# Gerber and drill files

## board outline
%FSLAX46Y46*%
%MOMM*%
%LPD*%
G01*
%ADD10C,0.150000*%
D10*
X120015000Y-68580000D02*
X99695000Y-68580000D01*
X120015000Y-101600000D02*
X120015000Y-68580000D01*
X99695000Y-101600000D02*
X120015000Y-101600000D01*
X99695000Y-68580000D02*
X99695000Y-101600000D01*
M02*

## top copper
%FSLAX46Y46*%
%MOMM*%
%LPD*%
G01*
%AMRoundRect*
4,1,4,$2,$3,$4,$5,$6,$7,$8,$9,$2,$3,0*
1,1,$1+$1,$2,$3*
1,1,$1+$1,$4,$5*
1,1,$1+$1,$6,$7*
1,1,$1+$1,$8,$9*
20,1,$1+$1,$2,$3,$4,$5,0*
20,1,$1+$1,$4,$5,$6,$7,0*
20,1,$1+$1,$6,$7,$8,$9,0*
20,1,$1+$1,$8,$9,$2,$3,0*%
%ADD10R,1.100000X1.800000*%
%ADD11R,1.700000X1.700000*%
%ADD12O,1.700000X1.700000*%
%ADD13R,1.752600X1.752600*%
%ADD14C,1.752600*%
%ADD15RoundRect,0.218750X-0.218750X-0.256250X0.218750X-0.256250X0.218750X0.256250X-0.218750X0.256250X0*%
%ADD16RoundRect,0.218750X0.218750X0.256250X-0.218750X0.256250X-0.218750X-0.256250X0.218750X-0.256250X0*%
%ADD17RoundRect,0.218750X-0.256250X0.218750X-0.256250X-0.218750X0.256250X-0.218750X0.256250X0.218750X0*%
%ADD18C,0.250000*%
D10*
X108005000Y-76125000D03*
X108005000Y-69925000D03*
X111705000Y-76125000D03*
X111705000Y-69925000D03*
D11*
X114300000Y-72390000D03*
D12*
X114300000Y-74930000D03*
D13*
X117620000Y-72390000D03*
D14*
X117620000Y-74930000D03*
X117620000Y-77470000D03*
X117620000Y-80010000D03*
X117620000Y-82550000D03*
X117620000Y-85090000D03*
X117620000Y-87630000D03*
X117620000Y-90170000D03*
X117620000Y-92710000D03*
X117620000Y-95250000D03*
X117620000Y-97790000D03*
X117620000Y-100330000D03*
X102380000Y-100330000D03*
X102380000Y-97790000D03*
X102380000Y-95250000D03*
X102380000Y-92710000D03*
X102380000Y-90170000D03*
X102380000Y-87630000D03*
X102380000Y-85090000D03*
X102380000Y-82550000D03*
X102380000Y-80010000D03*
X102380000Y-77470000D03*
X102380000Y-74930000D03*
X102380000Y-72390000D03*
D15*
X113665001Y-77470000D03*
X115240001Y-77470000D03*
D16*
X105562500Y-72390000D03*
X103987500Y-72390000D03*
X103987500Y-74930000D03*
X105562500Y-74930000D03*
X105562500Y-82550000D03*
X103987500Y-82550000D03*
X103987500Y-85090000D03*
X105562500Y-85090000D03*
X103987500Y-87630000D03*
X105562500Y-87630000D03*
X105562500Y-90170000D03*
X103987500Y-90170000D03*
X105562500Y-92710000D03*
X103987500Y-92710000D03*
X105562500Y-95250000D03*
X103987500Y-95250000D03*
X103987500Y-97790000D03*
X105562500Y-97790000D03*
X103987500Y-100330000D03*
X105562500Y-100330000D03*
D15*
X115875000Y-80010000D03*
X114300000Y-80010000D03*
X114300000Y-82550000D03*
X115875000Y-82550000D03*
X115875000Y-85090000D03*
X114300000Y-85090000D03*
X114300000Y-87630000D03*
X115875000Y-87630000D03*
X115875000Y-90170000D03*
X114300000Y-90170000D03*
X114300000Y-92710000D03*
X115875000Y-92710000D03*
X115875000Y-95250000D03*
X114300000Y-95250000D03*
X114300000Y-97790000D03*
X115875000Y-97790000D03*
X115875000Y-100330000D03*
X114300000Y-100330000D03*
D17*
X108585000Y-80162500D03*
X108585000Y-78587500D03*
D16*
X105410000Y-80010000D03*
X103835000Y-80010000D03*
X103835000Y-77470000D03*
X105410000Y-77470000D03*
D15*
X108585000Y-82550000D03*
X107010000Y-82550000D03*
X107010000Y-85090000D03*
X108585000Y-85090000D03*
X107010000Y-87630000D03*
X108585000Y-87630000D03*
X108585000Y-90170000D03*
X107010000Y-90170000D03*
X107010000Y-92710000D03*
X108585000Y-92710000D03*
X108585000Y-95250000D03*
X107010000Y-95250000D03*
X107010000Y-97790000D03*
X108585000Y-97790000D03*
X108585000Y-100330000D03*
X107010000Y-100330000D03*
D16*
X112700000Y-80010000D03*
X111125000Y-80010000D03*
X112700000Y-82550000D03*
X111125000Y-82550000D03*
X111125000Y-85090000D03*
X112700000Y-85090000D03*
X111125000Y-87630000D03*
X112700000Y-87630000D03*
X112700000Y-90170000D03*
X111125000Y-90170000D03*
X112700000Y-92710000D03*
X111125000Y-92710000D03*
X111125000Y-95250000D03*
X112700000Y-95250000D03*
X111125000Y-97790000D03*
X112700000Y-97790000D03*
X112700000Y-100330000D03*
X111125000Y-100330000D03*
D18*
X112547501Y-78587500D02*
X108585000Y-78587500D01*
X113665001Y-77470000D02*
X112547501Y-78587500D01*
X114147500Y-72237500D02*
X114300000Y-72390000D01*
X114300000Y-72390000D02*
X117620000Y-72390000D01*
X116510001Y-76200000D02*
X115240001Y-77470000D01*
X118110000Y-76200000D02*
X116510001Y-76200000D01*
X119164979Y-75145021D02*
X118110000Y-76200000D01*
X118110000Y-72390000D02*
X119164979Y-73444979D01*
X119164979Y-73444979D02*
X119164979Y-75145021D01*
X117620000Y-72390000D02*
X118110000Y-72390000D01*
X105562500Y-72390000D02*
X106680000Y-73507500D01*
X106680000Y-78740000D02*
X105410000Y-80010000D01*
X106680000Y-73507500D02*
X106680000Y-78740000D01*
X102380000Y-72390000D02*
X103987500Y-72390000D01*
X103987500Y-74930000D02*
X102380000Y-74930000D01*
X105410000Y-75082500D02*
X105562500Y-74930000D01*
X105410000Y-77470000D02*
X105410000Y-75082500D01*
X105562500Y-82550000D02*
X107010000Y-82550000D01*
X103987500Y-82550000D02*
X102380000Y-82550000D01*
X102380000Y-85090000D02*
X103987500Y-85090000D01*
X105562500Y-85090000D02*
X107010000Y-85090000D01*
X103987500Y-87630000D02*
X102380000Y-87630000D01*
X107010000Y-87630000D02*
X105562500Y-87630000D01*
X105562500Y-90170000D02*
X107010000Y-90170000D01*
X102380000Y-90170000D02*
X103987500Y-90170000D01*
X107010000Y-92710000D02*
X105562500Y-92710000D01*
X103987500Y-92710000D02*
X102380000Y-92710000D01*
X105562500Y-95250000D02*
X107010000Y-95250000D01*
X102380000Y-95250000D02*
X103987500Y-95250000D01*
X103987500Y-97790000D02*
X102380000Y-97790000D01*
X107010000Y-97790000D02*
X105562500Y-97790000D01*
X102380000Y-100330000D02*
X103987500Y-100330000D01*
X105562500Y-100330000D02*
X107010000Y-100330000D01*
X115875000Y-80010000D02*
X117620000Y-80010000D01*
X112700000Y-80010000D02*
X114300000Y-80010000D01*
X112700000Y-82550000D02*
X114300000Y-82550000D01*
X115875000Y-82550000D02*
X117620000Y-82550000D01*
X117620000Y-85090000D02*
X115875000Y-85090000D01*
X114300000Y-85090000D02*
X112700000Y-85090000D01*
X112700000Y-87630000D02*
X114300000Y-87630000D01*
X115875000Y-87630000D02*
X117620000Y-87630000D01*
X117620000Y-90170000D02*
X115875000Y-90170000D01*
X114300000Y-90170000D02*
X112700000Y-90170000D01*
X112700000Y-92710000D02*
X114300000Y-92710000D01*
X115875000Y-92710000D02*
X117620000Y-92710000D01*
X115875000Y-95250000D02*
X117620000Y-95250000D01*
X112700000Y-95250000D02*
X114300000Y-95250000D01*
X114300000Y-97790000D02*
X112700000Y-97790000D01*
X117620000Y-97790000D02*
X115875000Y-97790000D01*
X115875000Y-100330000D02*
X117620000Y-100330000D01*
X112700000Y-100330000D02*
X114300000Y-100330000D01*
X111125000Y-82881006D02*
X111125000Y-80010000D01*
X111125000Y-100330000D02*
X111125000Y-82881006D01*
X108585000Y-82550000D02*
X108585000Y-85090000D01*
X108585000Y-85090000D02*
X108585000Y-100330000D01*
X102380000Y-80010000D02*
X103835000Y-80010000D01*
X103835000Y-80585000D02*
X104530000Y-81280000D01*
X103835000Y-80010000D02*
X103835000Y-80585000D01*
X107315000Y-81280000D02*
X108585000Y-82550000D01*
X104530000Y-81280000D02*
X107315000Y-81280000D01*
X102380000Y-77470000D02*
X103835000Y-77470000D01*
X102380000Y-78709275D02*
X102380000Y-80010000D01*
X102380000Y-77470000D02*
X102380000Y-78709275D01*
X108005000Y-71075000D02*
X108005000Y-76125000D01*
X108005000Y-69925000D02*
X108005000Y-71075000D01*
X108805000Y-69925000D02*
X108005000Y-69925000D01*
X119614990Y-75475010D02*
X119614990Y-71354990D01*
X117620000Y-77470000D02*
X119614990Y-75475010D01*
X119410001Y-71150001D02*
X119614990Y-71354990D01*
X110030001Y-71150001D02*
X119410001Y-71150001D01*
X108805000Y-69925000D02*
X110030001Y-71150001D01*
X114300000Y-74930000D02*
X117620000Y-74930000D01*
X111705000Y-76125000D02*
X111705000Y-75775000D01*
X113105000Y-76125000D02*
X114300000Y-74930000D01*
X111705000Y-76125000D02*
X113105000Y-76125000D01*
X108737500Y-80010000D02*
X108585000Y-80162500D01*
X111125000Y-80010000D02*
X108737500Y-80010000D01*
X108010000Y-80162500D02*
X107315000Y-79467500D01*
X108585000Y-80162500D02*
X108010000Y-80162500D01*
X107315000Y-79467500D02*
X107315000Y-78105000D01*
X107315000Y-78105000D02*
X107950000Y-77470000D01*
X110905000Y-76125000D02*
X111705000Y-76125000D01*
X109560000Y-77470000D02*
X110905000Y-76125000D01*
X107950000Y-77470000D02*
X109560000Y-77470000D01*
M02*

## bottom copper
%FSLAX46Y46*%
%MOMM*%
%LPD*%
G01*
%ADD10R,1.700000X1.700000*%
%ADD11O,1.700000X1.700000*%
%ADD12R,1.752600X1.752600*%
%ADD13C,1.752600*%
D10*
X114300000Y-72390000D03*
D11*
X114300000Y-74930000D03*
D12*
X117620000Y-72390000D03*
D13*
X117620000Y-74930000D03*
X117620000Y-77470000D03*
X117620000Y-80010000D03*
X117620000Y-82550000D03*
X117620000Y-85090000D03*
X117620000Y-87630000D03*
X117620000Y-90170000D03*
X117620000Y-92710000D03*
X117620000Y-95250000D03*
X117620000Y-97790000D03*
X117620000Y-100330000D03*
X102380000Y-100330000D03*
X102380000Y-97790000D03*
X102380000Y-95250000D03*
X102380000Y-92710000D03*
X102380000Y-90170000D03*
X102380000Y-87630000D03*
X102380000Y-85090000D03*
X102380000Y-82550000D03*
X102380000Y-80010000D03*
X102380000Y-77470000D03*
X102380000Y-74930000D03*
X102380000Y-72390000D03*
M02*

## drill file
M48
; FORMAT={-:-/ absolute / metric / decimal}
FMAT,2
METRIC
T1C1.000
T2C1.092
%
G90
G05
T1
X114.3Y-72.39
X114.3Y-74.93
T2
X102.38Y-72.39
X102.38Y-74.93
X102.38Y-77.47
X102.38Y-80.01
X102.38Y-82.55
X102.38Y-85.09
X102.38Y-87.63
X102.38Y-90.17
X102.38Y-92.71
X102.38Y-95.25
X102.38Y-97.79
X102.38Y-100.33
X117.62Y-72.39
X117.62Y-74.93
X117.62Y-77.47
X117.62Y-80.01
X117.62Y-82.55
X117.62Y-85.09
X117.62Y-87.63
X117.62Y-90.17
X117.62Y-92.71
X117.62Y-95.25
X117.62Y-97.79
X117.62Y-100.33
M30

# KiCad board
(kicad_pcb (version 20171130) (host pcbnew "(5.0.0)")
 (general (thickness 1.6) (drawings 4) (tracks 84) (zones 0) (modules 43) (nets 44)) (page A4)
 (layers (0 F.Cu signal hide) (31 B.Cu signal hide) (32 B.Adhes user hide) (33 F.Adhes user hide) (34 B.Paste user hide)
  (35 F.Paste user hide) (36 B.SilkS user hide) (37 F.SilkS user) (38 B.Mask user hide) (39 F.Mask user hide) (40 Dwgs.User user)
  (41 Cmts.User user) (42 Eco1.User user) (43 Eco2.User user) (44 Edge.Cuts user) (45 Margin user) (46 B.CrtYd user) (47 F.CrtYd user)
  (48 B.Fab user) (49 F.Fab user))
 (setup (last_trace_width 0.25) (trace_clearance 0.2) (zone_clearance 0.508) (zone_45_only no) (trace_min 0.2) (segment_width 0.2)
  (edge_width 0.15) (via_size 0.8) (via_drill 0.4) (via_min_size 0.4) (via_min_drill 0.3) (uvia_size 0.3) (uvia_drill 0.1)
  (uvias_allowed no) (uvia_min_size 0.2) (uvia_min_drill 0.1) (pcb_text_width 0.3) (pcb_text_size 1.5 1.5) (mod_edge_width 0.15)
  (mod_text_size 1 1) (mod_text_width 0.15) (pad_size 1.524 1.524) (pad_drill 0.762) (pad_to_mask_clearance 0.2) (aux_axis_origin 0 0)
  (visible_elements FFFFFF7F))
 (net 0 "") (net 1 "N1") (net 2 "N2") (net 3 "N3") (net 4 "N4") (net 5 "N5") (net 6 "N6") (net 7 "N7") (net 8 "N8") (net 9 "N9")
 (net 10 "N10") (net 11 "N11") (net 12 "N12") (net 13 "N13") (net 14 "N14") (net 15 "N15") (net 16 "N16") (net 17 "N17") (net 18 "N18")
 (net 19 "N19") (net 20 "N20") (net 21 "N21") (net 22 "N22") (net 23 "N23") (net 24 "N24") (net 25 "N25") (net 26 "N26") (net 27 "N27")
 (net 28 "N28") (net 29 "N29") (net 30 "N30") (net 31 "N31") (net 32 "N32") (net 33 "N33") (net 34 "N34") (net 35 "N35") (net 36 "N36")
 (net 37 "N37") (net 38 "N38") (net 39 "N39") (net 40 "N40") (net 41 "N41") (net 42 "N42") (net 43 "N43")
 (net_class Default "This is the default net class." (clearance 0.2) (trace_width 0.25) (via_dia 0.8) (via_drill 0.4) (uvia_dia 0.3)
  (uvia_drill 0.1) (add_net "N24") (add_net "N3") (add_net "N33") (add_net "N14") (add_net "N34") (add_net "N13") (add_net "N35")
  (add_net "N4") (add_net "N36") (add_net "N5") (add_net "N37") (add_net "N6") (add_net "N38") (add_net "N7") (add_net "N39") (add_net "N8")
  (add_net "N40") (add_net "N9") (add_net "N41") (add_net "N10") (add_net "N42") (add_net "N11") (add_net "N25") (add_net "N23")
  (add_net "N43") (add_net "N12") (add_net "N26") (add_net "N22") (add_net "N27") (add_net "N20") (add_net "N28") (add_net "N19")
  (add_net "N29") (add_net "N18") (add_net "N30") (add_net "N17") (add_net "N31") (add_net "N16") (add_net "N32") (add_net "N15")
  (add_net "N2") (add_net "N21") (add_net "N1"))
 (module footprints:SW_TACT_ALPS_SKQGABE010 (layer F.Cu) (at 109.855 73.025 90)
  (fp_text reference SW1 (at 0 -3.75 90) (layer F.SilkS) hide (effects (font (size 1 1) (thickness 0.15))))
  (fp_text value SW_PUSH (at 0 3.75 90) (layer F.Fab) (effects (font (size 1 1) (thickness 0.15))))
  (pad 1 smd rect (at -3.1 -1.85 90) (size 1.8 1.1) (layers F.Cu F.Paste F.Mask) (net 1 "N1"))
  (pad 1 smd rect (at 3.1 -1.85 90) (size 1.8 1.1) (layers F.Cu F.Paste F.Mask) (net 1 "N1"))
  (pad 2 smd rect (at -3.1 1.85 90) (size 1.8 1.1) (layers F.Cu F.Paste F.Mask) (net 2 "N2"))
  (pad 2 smd rect (at 3.1 1.85 90) (size 1.8 1.1) (layers F.Cu F.Paste F.Mask) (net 2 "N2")))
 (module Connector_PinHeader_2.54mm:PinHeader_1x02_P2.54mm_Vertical (layer F.Cu) (at 114.3 72.39)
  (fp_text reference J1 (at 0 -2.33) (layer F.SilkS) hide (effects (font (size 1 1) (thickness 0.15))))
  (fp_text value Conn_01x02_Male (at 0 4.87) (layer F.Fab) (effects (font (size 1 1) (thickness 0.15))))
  (pad 1 thru_hole rect (at 0 0) (size 1.7 1.7) (drill 1) (layers *.Cu *.Mask) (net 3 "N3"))
  (pad 2 thru_hole oval (at 0 2.54) (size 1.7 1.7) (drill 1) (layers *.Cu *.Mask) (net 2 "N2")))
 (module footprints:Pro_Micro (layer B.Cu) (at 110 84.836 180)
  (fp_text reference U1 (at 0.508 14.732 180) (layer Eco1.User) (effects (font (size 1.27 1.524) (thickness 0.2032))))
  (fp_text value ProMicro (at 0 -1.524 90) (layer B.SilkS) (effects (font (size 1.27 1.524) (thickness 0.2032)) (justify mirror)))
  (pad 1 thru_hole rect (at -7.62 12.446 270) (size 1.7526 1.7526) (drill 1.0922) (layers *.Cu *.SilkS *.Mask) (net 3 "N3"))
  (pad 2 thru_hole circle (at -7.62 9.906 270) (size 1.7526 1.7526) (drill 1.0922) (layers *.Cu *.SilkS *.Mask) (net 2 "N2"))
  (pad 3 thru_hole circle (at -7.62 7.366 270) (size 1.7526 1.7526) (drill 1.0922) (layers *.Cu *.SilkS *.Mask) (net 1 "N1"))
  (pad 4 thru_hole circle (at -7.62 4.826 270) (size 1.7526 1.7526) (drill 1.0922) (layers *.Cu *.SilkS *.Mask) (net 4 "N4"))
  (pad 5 thru_hole circle (at -7.62 2.286 270) (size 1.7526 1.7526) (drill 1.0922) (layers *.Cu *.SilkS *.Mask) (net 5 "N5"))
  (pad 6 thru_hole circle (at -7.62 -0.254 270) (size 1.7526 1.7526) (drill 1.0922) (layers *.Cu *.SilkS *.Mask) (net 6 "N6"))
  (pad 7 thru_hole circle (at -7.62 -2.794 270) (size 1.7526 1.7526) (drill 1.0922) (layers *.Cu *.SilkS *.Mask) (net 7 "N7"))
  (pad 8 thru_hole circle (at -7.62 -5.334 270) (size 1.7526 1.7526) (drill 1.0922) (layers *.Cu *.SilkS *.Mask) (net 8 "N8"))
  (pad 9 thru_hole circle (at -7.62 -7.874 270) (size 1.7526 1.7526) (drill 1.0922) (layers *.Cu *.SilkS *.Mask) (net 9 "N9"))
  (pad 10 thru_hole circle (at -7.62 -10.414 270) (size 1.7526 1.7526) (drill 1.0922) (layers *.Cu *.SilkS *.Mask) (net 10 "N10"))
  (pad 11 thru_hole circle (at -7.62 -12.954 270) (size 1.7526 1.7526) (drill 1.0922) (layers *.Cu *.SilkS *.Mask) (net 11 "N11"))
  (pad 12 thru_hole circle (at -7.62 -15.494 270) (size 1.7526 1.7526) (drill 1.0922) (layers *.Cu *.SilkS *.Mask) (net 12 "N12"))
  (pad 24 thru_hole circle (at 7.62 -15.494 270) (size 1.7526 1.7526) (drill 1.0922) (layers *.Cu *.SilkS *.Mask) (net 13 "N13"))
  (pad 23 thru_hole circle (at 7.62 -12.954 270) (size 1.7526 1.7526) (drill 1.0922) (layers *.Cu *.SilkS *.Mask) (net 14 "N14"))
  (pad 22 thru_hole circle (at 7.62 -10.414 270) (size 1.7526 1.7526) (drill 1.0922) (layers *.Cu *.SilkS *.Mask) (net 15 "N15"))
  (pad 21 thru_hole circle (at 7.62 -7.874 270) (size 1.7526 1.7526) (drill 1.0922) (layers *.Cu *.SilkS *.Mask) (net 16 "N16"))
  (pad 20 thru_hole circle (at 7.62 -5.334 270) (size 1.7526 1.7526) (drill 1.0922) (layers *.Cu *.SilkS *.Mask) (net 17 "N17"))
  (pad 19 thru_hole circle (at 7.62 -2.794 270) (size 1.7526 1.7526) (drill 1.0922) (layers *.Cu *.SilkS *.Mask) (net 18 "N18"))
  (pad 18 thru_hole circle (at 7.62 -0.254 270) (size 1.7526 1.7526) (drill 1.0922) (layers *.Cu *.SilkS *.Mask) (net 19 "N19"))
  (pad 17 thru_hole circle (at 7.62 2.286 270) (size 1.7526 1.7526) (drill 1.0922) (layers *.Cu *.SilkS *.Mask) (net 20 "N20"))
  (pad 16 thru_hole circle (at 7.62 4.826 270) (size 1.7526 1.7526) (drill 1.0922) (layers *.Cu *.SilkS *.Mask) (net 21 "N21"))
  (pad 15 thru_hole circle (at 7.62 7.366 270) (size 1.7526 1.7526) (drill 1.0922) (layers *.Cu *.SilkS *.Mask) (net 21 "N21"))
  (pad 14 thru_hole circle (at 7.62 9.906 270) (size 1.7526 1.7526) (drill 1.0922) (layers *.Cu *.SilkS *.Mask) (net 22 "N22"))
  (pad 13 thru_hole circle (at 7.62 12.446 270) (size 1.7526 1.7526) (drill 1.0922) (layers *.Cu *.SilkS *.Mask) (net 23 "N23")))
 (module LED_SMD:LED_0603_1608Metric (layer F.Cu) (at 114.452501 77.47)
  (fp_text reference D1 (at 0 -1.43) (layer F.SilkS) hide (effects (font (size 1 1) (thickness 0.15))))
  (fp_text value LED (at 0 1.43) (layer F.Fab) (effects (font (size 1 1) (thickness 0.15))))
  (pad 1 smd roundrect (at -0.7875 0) (size 0.875 0.95) (layers F.Cu F.Paste F.Mask) (roundrect_rratio 0.25) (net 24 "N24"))
  (pad 2 smd roundrect (at 0.7875 0) (size 0.875 0.95) (layers F.Cu F.Paste F.Mask) (roundrect_rratio 0.25) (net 3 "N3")))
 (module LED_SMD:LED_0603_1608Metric (layer F.Cu) (at 104.775 72.39 180)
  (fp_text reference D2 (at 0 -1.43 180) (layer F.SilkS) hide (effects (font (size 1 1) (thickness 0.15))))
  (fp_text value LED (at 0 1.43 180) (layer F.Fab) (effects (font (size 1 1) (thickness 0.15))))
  (pad 1 smd roundrect (at -0.7875 0 180) (size 0.875 0.95) (layers F.Cu F.Paste F.Mask) (roundrect_rratio 0.25) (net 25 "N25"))
  (pad 2 smd roundrect (at 0.7875 0 180) (size 0.875 0.95) (layers F.Cu F.Paste F.Mask) (roundrect_rratio 0.25) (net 23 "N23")))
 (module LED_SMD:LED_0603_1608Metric (layer F.Cu) (at 104.775 74.93 180)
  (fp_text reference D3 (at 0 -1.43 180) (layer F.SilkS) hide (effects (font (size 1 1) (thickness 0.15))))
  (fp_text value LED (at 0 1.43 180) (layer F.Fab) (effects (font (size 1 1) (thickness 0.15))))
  (pad 2 smd roundrect (at 0.7875 0 180) (size 0.875 0.95) (layers F.Cu F.Paste F.Mask) (roundrect_rratio 0.25) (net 22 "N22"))
  (pad 1 smd roundrect (at -0.7875 0 180) (size 0.875 0.95) (layers F.Cu F.Paste F.Mask) (roundrect_rratio 0.25) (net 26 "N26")))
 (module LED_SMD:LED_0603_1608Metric (layer F.Cu) (at 104.775 82.55 180)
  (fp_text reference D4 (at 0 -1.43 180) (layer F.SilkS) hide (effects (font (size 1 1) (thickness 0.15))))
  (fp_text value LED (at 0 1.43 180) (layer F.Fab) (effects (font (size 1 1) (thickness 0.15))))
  (pad 1 smd roundrect (at -0.7875 0 180) (size 0.875 0.95) (layers F.Cu F.Paste F.Mask) (roundrect_rratio 0.25) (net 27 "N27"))
  (pad 2 smd roundrect (at 0.7875 0 180) (size 0.875 0.95) (layers F.Cu F.Paste F.Mask) (roundrect_rratio 0.25) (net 20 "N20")))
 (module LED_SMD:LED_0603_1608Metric (layer F.Cu) (at 104.775 85.09 180)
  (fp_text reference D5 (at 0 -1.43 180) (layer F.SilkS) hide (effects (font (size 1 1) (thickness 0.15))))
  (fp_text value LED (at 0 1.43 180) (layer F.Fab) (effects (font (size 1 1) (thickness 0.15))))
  (pad 2 smd roundrect (at 0.7875 0 180) (size 0.875 0.95) (layers F.Cu F.Paste F.Mask) (roundrect_rratio 0.25) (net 19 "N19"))
  (pad 1 smd roundrect (at -0.7875 0 180) (size 0.875 0.95) (layers F.Cu F.Paste F.Mask) (roundrect_rratio 0.25) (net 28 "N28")))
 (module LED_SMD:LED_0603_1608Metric (layer F.Cu) (at 104.775 87.63 180)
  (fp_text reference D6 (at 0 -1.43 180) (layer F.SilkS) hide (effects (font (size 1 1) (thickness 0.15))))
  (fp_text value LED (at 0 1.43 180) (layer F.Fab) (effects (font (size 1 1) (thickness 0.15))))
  (pad 2 smd roundrect (at 0.7875 0 180) (size 0.875 0.95) (layers F.Cu F.Paste F.Mask) (roundrect_rratio 0.25) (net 18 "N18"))
  (pad 1 smd roundrect (at -0.7875 0 180) (size 0.875 0.95) (layers F.Cu F.Paste F.Mask) (roundrect_rratio 0.25) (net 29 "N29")))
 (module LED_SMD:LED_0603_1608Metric (layer F.Cu) (at 104.775 90.17 180)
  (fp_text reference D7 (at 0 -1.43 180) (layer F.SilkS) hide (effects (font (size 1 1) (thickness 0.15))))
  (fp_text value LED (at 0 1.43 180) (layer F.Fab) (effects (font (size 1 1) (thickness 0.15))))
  (pad 1 smd roundrect (at -0.7875 0 180) (size 0.875 0.95) (layers F.Cu F.Paste F.Mask) (roundrect_rratio 0.25) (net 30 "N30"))
  (pad 2 smd roundrect (at 0.7875 0 180) (size 0.875 0.95) (layers F.Cu F.Paste F.Mask) (roundrect_rratio 0.25) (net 17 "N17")))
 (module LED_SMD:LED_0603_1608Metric (layer F.Cu) (at 104.775 92.71 180)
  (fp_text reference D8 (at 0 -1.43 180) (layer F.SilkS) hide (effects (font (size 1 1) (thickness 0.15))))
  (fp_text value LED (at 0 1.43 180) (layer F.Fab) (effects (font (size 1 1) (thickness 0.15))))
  (pad 1 smd roundrect (at -0.7875 0 180) (size 0.875 0.95) (layers F.Cu F.Paste F.Mask) (roundrect_rratio 0.25) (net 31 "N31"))
  (pad 2 smd roundrect (at 0.7875 0 180) (size 0.875 0.95) (layers F.Cu F.Paste F.Mask) (roundrect_rratio 0.25) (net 16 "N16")))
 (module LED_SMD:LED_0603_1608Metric (layer F.Cu) (at 104.775 95.25 180)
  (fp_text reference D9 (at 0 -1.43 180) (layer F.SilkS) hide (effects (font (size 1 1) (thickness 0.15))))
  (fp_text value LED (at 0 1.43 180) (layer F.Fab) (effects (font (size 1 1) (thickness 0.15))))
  (pad 1 smd roundrect (at -0.7875 0 180) (size 0.875 0.95) (layers F.Cu F.Paste F.Mask) (roundrect_rratio 0.25) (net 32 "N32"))
  (pad 2 smd roundrect (at 0.7875 0 180) (size 0.875 0.95) (layers F.Cu F.Paste F.Mask) (roundrect_rratio 0.25) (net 15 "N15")))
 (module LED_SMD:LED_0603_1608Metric (layer F.Cu) (at 104.775 97.79 180)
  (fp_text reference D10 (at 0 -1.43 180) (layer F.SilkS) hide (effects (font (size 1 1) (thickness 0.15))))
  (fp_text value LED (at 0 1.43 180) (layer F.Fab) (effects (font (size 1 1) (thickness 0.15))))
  (pad 2 smd roundrect (at 0.7875 0 180) (size 0.875 0.95) (layers F.Cu F.Paste F.Mask) (roundrect_rratio 0.25) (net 14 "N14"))
  (pad 1 smd roundrect (at -0.7875 0 180) (size 0.875 0.95) (layers F.Cu F.Paste F.Mask) (roundrect_rratio 0.25) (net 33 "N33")))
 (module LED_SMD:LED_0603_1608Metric (layer F.Cu) (at 104.775 100.33 180)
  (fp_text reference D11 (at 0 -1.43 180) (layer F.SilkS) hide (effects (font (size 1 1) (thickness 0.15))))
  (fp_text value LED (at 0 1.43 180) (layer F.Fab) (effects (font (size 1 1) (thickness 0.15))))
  (pad 2 smd roundrect (at 0.7875 0 180) (size 0.875 0.95) (layers F.Cu F.Paste F.Mask) (roundrect_rratio 0.25) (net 13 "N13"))
  (pad 1 smd roundrect (at -0.7875 0 180) (size 0.875 0.95) (layers F.Cu F.Paste F.Mask) (roundrect_rratio 0.25) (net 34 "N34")))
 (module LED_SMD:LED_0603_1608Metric (layer F.Cu) (at 115.0875 80.01)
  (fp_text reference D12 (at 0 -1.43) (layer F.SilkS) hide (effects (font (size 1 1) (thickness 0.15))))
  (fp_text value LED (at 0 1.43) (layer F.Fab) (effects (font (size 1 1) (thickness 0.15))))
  (pad 2 smd roundrect (at 0.7875 0) (size 0.875 0.95) (layers F.Cu F.Paste F.Mask) (roundrect_rratio 0.25) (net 4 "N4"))
  (pad 1 smd roundrect (at -0.7875 0) (size 0.875 0.95) (layers F.Cu F.Paste F.Mask) (roundrect_rratio 0.25) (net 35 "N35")))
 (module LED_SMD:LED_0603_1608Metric (layer F.Cu) (at 115.0875 82.55)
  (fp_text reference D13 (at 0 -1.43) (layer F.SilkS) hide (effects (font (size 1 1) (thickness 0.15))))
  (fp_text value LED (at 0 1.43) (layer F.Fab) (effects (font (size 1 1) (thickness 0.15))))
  (pad 1 smd roundrect (at -0.7875 0) (size 0.875 0.95) (layers F.Cu F.Paste F.Mask) (roundrect_rratio 0.25) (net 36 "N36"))
  (pad 2 smd roundrect (at 0.7875 0) (size 0.875 0.95) (layers F.Cu F.Paste F.Mask) (roundrect_rratio 0.25) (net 5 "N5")))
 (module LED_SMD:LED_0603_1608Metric (layer F.Cu) (at 115.0875 85.09)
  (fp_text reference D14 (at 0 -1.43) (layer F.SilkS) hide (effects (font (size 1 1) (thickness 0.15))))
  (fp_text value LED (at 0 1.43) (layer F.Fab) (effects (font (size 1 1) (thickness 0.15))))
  (pad 2 smd roundrect (at 0.7875 0) (size 0.875 0.95) (layers F.Cu F.Paste F.Mask) (roundrect_rratio 0.25) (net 6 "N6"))
  (pad 1 smd roundrect (at -0.7875 0) (size 0.875 0.95) (layers F.Cu F.Paste F.Mask) (roundrect_rratio 0.25) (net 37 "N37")))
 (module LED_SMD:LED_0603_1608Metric (layer F.Cu) (at 115.0875 87.63)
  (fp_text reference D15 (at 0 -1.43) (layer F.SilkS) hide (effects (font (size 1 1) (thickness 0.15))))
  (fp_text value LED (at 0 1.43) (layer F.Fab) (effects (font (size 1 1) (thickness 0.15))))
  (pad 1 smd roundrect (at -0.7875 0) (size 0.875 0.95) (layers F.Cu F.Paste F.Mask) (roundrect_rratio 0.25) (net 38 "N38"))
  (pad 2 smd roundrect (at 0.7875 0) (size 0.875 0.95) (layers F.Cu F.Paste F.Mask) (roundrect_rratio 0.25) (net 7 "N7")))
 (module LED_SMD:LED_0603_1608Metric (layer F.Cu) (at 115.0875 90.17)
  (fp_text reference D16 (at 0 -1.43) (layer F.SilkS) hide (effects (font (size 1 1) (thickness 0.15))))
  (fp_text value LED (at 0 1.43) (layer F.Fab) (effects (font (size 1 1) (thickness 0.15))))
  (pad 2 smd roundrect (at 0.7875 0) (size 0.875 0.95) (layers F.Cu F.Paste F.Mask) (roundrect_rratio 0.25) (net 8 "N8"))
  (pad 1 smd roundrect (at -0.7875 0) (size 0.875 0.95) (layers F.Cu F.Paste F.Mask) (roundrect_rratio 0.25) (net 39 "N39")))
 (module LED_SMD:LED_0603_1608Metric (layer F.Cu) (at 115.0875 92.71)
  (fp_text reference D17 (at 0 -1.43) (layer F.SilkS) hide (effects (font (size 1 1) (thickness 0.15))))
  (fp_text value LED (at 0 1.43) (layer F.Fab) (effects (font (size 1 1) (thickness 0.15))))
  (pad 1 smd roundrect (at -0.7875 0) (size 0.875 0.95) (layers F.Cu F.Paste F.Mask) (roundrect_rratio 0.25) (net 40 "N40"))
  (pad 2 smd roundrect (at 0.7875 0) (size 0.875 0.95) (layers F.Cu F.Paste F.Mask) (roundrect_rratio 0.25) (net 9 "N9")))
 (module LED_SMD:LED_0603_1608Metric (layer F.Cu) (at 115.0875 95.25)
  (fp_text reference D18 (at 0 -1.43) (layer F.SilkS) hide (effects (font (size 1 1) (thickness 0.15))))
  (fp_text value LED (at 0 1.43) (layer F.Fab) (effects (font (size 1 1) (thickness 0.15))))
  (pad 2 smd roundrect (at 0.7875 0) (size 0.875 0.95) (layers F.Cu F.Paste F.Mask) (roundrect_rratio 0.25) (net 10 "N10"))
  (pad 1 smd roundrect (at -0.7875 0) (size 0.875 0.95) (layers F.Cu F.Paste F.Mask) (roundrect_rratio 0.25) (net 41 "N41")))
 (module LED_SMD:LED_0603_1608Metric (layer F.Cu) (at 115.0875 97.79)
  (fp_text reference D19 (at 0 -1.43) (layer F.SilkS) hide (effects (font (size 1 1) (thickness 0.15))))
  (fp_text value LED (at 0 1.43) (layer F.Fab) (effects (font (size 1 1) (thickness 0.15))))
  (pad 1 smd roundrect (at -0.7875 0) (size 0.875 0.95) (layers F.Cu F.Paste F.Mask) (roundrect_rratio 0.25) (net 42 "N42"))
  (pad 2 smd roundrect (at 0.7875 0) (size 0.875 0.95) (layers F.Cu F.Paste F.Mask) (roundrect_rratio 0.25) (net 11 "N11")))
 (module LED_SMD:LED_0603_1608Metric (layer F.Cu) (at 115.0875 100.33)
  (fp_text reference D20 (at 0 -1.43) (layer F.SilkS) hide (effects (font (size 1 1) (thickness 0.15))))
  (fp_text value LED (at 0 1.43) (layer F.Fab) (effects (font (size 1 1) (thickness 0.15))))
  (pad 2 smd roundrect (at 0.7875 0) (size 0.875 0.95) (layers F.Cu F.Paste F.Mask) (roundrect_rratio 0.25) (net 12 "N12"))
  (pad 1 smd roundrect (at -0.7875 0) (size 0.875 0.95) (layers F.Cu F.Paste F.Mask) (roundrect_rratio 0.25) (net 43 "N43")))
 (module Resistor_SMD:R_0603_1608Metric (layer F.Cu) (at 108.585 79.375 270)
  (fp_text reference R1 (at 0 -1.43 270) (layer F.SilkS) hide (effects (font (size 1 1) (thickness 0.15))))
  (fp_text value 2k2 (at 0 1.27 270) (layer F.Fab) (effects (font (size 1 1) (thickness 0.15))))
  (pad 2 smd roundrect (at 0.7875 0 270) (size 0.875 0.95) (layers F.Cu F.Paste F.Mask) (roundrect_rratio 0.25) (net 2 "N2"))
  (pad 1 smd roundrect (at -0.7875 0 270) (size 0.875 0.95) (layers F.Cu F.Paste F.Mask) (roundrect_rratio 0.25) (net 24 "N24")))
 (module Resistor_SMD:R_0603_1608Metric (layer F.Cu) (at 104.6225 80.01 180)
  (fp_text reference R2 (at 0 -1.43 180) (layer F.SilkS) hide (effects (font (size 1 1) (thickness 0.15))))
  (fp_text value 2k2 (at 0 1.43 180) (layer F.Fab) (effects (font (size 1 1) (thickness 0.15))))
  (pad 1 smd roundrect (at -0.7875 0 180) (size 0.875 0.95) (layers F.Cu F.Paste F.Mask) (roundrect_rratio 0.25) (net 25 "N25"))
  (pad 2 smd roundrect (at 0.7875 0 180) (size 0.875 0.95) (layers F.Cu F.Paste F.Mask) (roundrect_rratio 0.25) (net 21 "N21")))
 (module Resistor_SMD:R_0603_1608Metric (layer F.Cu) (at 104.6225 77.47 180)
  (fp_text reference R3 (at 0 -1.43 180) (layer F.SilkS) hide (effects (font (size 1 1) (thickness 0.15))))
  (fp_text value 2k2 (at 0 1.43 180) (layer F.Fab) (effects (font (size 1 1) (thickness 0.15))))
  (pad 2 smd roundrect (at 0.7875 0 180) (size 0.875 0.95) (layers F.Cu F.Paste F.Mask) (roundrect_rratio 0.25) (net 21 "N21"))
  (pad 1 smd roundrect (at -0.7875 0 180) (size 0.875 0.95) (layers F.Cu F.Paste F.Mask) (roundrect_rratio 0.25) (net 26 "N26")))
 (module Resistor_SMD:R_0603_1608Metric (layer F.Cu) (at 107.7975 82.55)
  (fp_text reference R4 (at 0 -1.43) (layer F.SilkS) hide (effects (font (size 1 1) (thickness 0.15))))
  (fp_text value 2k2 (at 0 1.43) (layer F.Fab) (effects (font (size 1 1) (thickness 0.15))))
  (pad 2 smd roundrect (at 0.7875 0) (size 0.875 0.95) (layers F.Cu F.Paste F.Mask) (roundrect_rratio 0.25) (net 21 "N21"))
  (pad 1 smd roundrect (at -0.7875 0) (size 0.875 0.95) (layers F.Cu F.Paste F.Mask) (roundrect_rratio 0.25) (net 27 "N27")))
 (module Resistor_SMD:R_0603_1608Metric (layer F.Cu) (at 107.7975 85.09)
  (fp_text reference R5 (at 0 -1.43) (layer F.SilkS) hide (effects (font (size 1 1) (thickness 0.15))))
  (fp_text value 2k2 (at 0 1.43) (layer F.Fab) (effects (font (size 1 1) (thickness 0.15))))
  (pad 1 smd roundrect (at -0.7875 0) (size 0.875 0.95) (layers F.Cu F.Paste F.Mask) (roundrect_rratio 0.25) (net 28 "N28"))
  (pad 2 smd roundrect (at 0.7875 0) (size 0.875 0.95) (layers F.Cu F.Paste F.Mask) (roundrect_rratio 0.25) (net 21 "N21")))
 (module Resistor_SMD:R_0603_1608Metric (layer F.Cu) (at 107.7975 87.63)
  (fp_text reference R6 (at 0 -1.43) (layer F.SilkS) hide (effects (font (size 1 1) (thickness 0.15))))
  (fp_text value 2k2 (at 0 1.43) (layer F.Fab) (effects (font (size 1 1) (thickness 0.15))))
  (pad 1 smd roundrect (at -0.7875 0) (size 0.875 0.95) (layers F.Cu F.Paste F.Mask) (roundrect_rratio 0.25) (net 29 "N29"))
  (pad 2 smd roundrect (at 0.7875 0) (size 0.875 0.95) (layers F.Cu F.Paste F.Mask) (roundrect_rratio 0.25) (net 21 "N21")))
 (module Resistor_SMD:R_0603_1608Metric (layer F.Cu) (at 107.7975 90.17)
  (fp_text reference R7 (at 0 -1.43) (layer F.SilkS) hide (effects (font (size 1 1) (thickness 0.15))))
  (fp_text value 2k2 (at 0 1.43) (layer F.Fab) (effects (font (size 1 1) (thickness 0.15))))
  (pad 2 smd roundrect (at 0.7875 0) (size 0.875 0.95) (layers F.Cu F.Paste F.Mask) (roundrect_rratio 0.25) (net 21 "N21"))
  (pad 1 smd roundrect (at -0.7875 0) (size 0.875 0.95) (layers F.Cu F.Paste F.Mask) (roundrect_rratio 0.25) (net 30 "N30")))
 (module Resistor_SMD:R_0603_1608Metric (layer F.Cu) (at 107.7975 92.71)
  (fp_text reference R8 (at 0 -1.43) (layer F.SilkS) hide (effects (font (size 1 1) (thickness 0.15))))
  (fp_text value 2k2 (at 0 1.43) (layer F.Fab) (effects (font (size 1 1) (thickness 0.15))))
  (pad 1 smd roundrect (at -0.7875 0) (size 0.875 0.95) (layers F.Cu F.Paste F.Mask) (roundrect_rratio 0.25) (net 31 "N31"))
  (pad 2 smd roundrect (at 0.7875 0) (size 0.875 0.95) (layers F.Cu F.Paste F.Mask) (roundrect_rratio 0.25) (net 21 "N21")))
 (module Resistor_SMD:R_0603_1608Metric (layer F.Cu) (at 107.7975 95.25)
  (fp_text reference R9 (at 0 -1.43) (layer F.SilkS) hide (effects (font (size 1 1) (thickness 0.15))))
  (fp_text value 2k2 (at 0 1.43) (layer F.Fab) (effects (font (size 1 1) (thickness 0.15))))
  (pad 2 smd roundrect (at 0.7875 0) (size 0.875 0.95) (layers F.Cu F.Paste F.Mask) (roundrect_rratio 0.25) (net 21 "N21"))
  (pad 1 smd roundrect (at -0.7875 0) (size 0.875 0.95) (layers F.Cu F.Paste F.Mask) (roundrect_rratio 0.25) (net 32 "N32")))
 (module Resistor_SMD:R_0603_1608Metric (layer F.Cu) (at 107.7975 97.79)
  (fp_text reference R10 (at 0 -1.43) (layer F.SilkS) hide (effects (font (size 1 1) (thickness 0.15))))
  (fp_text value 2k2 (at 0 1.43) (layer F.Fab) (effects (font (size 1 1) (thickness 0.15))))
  (pad 1 smd roundrect (at -0.7875 0) (size 0.875 0.95) (layers F.Cu F.Paste F.Mask) (roundrect_rratio 0.25) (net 33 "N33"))
  (pad 2 smd roundrect (at 0.7875 0) (size 0.875 0.95) (layers F.Cu F.Paste F.Mask) (roundrect_rratio 0.25) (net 21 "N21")))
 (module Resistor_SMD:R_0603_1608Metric (layer F.Cu) (at 107.7975 100.33)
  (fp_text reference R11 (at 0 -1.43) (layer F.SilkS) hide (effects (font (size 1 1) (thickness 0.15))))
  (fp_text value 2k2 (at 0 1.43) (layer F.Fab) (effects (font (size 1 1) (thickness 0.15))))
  (pad 2 smd roundrect (at 0.7875 0) (size 0.875 0.95) (layers F.Cu F.Paste F.Mask) (roundrect_rratio 0.25) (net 21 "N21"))
  (pad 1 smd roundrect (at -0.7875 0) (size 0.875 0.95) (layers F.Cu F.Paste F.Mask) (roundrect_rratio 0.25) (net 34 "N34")))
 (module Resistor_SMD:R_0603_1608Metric (layer F.Cu) (at 111.9125 80.01 180)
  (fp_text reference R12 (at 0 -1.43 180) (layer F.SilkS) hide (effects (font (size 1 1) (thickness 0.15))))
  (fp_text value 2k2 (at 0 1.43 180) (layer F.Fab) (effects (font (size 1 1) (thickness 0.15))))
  (pad 1 smd roundrect (at -0.7875 0 180) (size 0.875 0.95) (layers F.Cu F.Paste F.Mask) (roundrect_rratio 0.25) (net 35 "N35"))
  (pad 2 smd roundrect (at 0.7875 0 180) (size 0.875 0.95) (layers F.Cu F.Paste F.Mask) (roundrect_rratio 0.25) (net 2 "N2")))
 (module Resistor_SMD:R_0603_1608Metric (layer F.Cu) (at 111.9125 82.55 180)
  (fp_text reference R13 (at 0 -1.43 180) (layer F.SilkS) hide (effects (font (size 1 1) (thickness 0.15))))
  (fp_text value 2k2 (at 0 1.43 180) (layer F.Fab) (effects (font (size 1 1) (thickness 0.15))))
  (pad 1 smd roundrect (at -0.7875 0 180) (size 0.875 0.95) (layers F.Cu F.Paste F.Mask) (roundrect_rratio 0.25) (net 36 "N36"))
  (pad 2 smd roundrect (at 0.7875 0 180) (size 0.875 0.95) (layers F.Cu F.Paste F.Mask) (roundrect_rratio 0.25) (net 2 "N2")))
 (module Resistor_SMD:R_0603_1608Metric (layer F.Cu) (at 111.9125 85.09 180)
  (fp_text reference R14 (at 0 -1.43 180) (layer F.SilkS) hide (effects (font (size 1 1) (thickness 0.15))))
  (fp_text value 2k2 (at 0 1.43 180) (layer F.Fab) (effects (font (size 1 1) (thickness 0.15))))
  (pad 2 smd roundrect (at 0.7875 0 180) (size 0.875 0.95) (layers F.Cu F.Paste F.Mask) (roundrect_rratio 0.25) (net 2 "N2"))
  (pad 1 smd roundrect (at -0.7875 0 180) (size 0.875 0.95) (layers F.Cu F.Paste F.Mask) (roundrect_rratio 0.25) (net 37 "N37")))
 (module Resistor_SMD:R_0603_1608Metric (layer F.Cu) (at 111.9125 87.63 180)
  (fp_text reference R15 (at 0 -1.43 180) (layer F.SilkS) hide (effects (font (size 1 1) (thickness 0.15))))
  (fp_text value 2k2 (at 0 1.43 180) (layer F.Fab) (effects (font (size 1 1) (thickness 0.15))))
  (pad 2 smd roundrect (at 0.7875 0 180) (size 0.875 0.95) (layers F.Cu F.Paste F.Mask) (roundrect_rratio 0.25) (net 2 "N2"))
  (pad 1 smd roundrect (at -0.7875 0 180) (size 0.875 0.95) (layers F.Cu F.Paste F.Mask) (roundrect_rratio 0.25) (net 38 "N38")))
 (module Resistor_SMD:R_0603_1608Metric (layer F.Cu) (at 111.9125 90.17 180)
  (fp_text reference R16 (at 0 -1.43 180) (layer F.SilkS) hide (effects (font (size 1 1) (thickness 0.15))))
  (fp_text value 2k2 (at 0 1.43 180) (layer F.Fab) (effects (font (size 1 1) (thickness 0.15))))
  (pad 1 smd roundrect (at -0.7875 0 180) (size 0.875 0.95) (layers F.Cu F.Paste F.Mask) (roundrect_rratio 0.25) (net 39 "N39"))
  (pad 2 smd roundrect (at 0.7875 0 180) (size 0.875 0.95) (layers F.Cu F.Paste F.Mask) (roundrect_rratio 0.25) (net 2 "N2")))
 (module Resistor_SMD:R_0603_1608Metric (layer F.Cu) (at 111.9125 92.71 180)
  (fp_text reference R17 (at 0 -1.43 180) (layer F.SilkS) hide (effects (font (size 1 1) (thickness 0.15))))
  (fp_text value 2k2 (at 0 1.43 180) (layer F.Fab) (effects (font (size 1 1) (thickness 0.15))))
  (pad 1 smd roundrect (at -0.7875 0 180) (size 0.875 0.95) (layers F.Cu F.Paste F.Mask) (roundrect_rratio 0.25) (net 40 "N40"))
  (pad 2 smd roundrect (at 0.7875 0 180) (size 0.875 0.95) (layers F.Cu F.Paste F.Mask) (roundrect_rratio 0.25) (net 2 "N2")))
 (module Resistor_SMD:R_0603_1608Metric (layer F.Cu) (at 111.9125 95.25 180)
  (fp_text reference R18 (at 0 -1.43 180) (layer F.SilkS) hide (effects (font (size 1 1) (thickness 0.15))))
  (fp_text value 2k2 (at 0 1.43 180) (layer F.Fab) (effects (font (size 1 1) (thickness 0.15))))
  (pad 2 smd roundrect (at 0.7875 0 180) (size 0.875 0.95) (layers F.Cu F.Paste F.Mask) (roundrect_rratio 0.25) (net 2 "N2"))
  (pad 1 smd roundrect (at -0.7875 0 180) (size 0.875 0.95) (layers F.Cu F.Paste F.Mask) (roundrect_rratio 0.25) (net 41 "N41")))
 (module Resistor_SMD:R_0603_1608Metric (layer F.Cu) (at 111.9125 97.79 180)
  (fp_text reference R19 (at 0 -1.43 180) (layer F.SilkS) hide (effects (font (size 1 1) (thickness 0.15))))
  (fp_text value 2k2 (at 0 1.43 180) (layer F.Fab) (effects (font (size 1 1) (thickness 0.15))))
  (pad 2 smd roundrect (at 0.7875 0 180) (size 0.875 0.95) (layers F.Cu F.Paste F.Mask) (roundrect_rratio 0.25) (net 2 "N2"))
  (pad 1 smd roundrect (at -0.7875 0 180) (size 0.875 0.95) (layers F.Cu F.Paste F.Mask) (roundrect_rratio 0.25) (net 42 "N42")))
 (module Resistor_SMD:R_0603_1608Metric (layer F.Cu) (at 111.9125 100.33 180)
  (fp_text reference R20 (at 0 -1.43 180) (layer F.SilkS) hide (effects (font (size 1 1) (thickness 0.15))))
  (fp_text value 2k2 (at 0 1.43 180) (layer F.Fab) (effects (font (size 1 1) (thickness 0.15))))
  (pad 1 smd roundrect (at -0.7875 0 180) (size 0.875 0.95) (layers F.Cu F.Paste F.Mask) (roundrect_rratio 0.25) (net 43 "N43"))
  (pad 2 smd roundrect (at 0.7875 0 180) (size 0.875 0.95) (layers F.Cu F.Paste F.Mask) (roundrect_rratio 0.25) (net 2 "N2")))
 (gr_line (start 120.015 68.58) (end 99.695 68.58) (layer Edge.Cuts) (width 0.15))
 (gr_line (start 120.015 101.6) (end 120.015 68.58) (layer Edge.Cuts) (width 0.15))
 (gr_line (start 99.695 101.6) (end 120.015 101.6) (layer Edge.Cuts) (width 0.15))
 (gr_line (start 99.695 68.58) (end 99.695 101.6) (layer Edge.Cuts) (width 0.15))
 (segment (start 112.547501 78.5875) (end 108.585 78.5875) (width 0.25) (layer F.Cu) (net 24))
 (segment (start 113.665001 77.47) (end 112.547501 78.5875) (width 0.25) (layer F.Cu) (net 24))
 (segment (start 114.1475 72.2375) (end 114.3 72.39) (width 0.25) (layer F.Cu) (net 3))
 (segment (start 114.3 72.39) (end 117.62 72.39) (width 0.25) (layer F.Cu) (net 3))
 (segment (start 116.510001 76.2) (end 115.240001 77.47) (width 0.25) (layer F.Cu) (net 3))
 (segment (start 118.11 76.2) (end 116.510001 76.2) (width 0.25) (layer F.Cu) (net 3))
 (segment (start 119.164979 75.145021) (end 118.11 76.2) (width 0.25) (layer F.Cu) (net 3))
 (segment (start 118.11 72.39) (end 119.164979 73.444979) (width 0.25) (layer F.Cu) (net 3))
 (segment (start 119.164979 73.444979) (end 119.164979 75.145021) (width 0.25) (layer F.Cu) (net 3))
 (segment (start 117.62 72.39) (end 118.11 72.39) (width 0.25) (layer F.Cu) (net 3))
 (segment (start 105.5625 72.39) (end 106.68 73.5075) (width 0.25) (layer F.Cu) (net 25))
 (segment (start 106.68 78.74) (end 105.41 80.01) (width 0.25) (layer F.Cu) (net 25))
 (segment (start 106.68 73.5075) (end 106.68 78.74) (width 0.25) (layer F.Cu) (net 25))
 (segment (start 102.38 72.39) (end 103.9875 72.39) (width 0.25) (layer F.Cu) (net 23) (status 30))
 (segment (start 103.9875 74.93) (end 102.38 74.93) (width 0.25) (layer F.Cu) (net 22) (status 30))
 (segment (start 105.41 75.0825) (end 105.5625 74.93) (width 0.25) (layer F.Cu) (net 26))
 (segment (start 105.41 77.47) (end 105.41 75.0825) (width 0.25) (layer F.Cu) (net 26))
 (segment (start 105.5625 82.55) (end 107.01 82.55) (width 0.25) (layer F.Cu) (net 27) (status 30))
 (segment (start 103.9875 82.55) (end 102.38 82.55) (width 0.25) (layer F.Cu) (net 20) (status 30))
 (segment (start 102.38 85.09) (end 103.9875 85.09) (width 0.25) (layer F.Cu) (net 19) (status 30))
 (segment (start 105.5625 85.09) (end 107.01 85.09) (width 0.25) (layer F.Cu) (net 28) (status 30))
 (segment (start 103.9875 87.63) (end 102.38 87.63) (width 0.25) (layer F.Cu) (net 18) (status 30))
 (segment (start 107.01 87.63) (end 105.5625 87.63) (width 0.25) (layer F.Cu) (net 29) (status 30))
 (segment (start 105.5625 90.17) (end 107.01 90.17) (width 0.25) (layer F.Cu) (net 30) (status 30))
 (segment (start 102.38 90.17) (end 103.9875 90.17) (width 0.25) (layer F.Cu) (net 17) (status 30))
 (segment (start 107.01 92.71) (end 105.5625 92.71) (width 0.25) (layer F.Cu) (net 31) (status 30))
 (segment (start 103.9875 92.71) (end 102.38 92.71) (width 0.25) (layer F.Cu) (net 16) (status 30))
 (segment (start 105.5625 95.25) (end 107.01 95.25) (width 0.25) (layer F.Cu) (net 32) (status 30))
 (segment (start 102.38 95.25) (end 103.9875 95.25) (width 0.25) (layer F.Cu) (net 15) (status 30))
 (segment (start 103.9875 97.79) (end 102.38 97.79) (width 0.25) (layer F.Cu) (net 14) (status 30))
 (segment (start 107.01 97.79) (end 105.5625 97.79) (width 0.25) (layer F.Cu) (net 33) (status 30))
 (segment (start 102.38 100.33) (end 103.9875 100.33) (width 0.25) (layer F.Cu) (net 13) (status 30))
 (segment (start 105.5625 100.33) (end 107.01 100.33) (width 0.25) (layer F.Cu) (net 34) (status 30))
 (segment (start 115.875 80.01) (end 117.62 80.01) (width 0.25) (layer F.Cu) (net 4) (status 30))
 (segment (start 112.7 80.01) (end 114.3 80.01) (width 0.25) (layer F.Cu) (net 35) (status 30))
 (segment (start 112.7 82.55) (end 114.3 82.55) (width 0.25) (layer F.Cu) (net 36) (status 30))
 (segment (start 115.875 82.55) (end 117.62 82.55) (width 0.25) (layer F.Cu) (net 5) (status 30))
 (segment (start 117.62 85.09) (end 115.875 85.09) (width 0.25) (layer F.Cu) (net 6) (status 30))
 (segment (start 114.3 85.09) (end 112.7 85.09) (width 0.25) (layer F.Cu) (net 37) (status 30))
 (segment (start 112.7 87.63) (end 114.3 87.63) (width 0.25) (layer F.Cu) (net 38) (status 30))
 (segment (start 115.875 87.63) (end 117.62 87.63) (width 0.25) (layer F.Cu) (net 7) (status 30))
 (segment (start 117.62 90.17) (end 115.875 90.17) (width 0.25) (layer F.Cu) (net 8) (status 30))
 (segment (start 114.3 90.17) (end 112.7 90.17) (width 0.25) (layer F.Cu) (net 39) (status 30))
 (segment (start 112.7 92.71) (end 114.3 92.71) (width 0.25) (layer F.Cu) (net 40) (status 30))
 (segment (start 115.875 92.71) (end 117.62 92.71) (width 0.25) (layer F.Cu) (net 9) (status 30))
 (segment (start 115.875 95.25) (end 117.62 95.25) (width 0.25) (layer F.Cu) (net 10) (status 30))
 (segment (start 112.7 95.25) (end 114.3 95.25) (width 0.25) (layer F.Cu) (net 41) (status 30))
 (segment (start 114.3 97.79) (end 112.7 97.79) (width 0.25) (layer F.Cu) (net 42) (status 30))
 (segment (start 117.62 97.79) (end 115.875 97.79) (width 0.25) (layer F.Cu) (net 11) (status 30))
 (segment (start 115.875 100.33) (end 117.62 100.33) (width 0.25) (layer F.Cu) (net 12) (status 30))
 (segment (start 112.7 100.33) (end 114.3 100.33) (width 0.25) (layer F.Cu) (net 43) (status 30))
 (segment (start 111.125 82.881006) (end 111.125 80.01) (width 0.25) (layer F.Cu) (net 2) (status 30))
 (segment (start 111.125 100.33) (end 111.125 82.881006) (width 0.25) (layer F.Cu) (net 2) (status 30))
 (segment (start 108.585 82.55) (end 108.585 85.09) (width 0.25) (layer F.Cu) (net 21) (status 30))
 (segment (start 108.585 85.09) (end 108.585 100.33) (width 0.25) (layer F.Cu) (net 21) (status 30))
 (segment (start 102.38 80.01) (end 103.835 80.01) (width 0.25) (layer F.Cu) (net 21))
 (segment (start 103.835 80.585) (end 104.53 81.28) (width 0.25) (layer F.Cu) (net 21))
 (segment (start 103.835 80.01) (end 103.835 80.585) (width 0.25) (layer F.Cu) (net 21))
 (segment (start 107.315 81.28) (end 108.585 82.55) (width 0.25) (layer F.Cu) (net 21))
 (segment (start 104.53 81.28) (end 107.315 81.28) (width 0.25) (layer F.Cu) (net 21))
 (segment (start 102.38 77.47) (end 103.835 77.47) (width 0.25) (layer F.Cu) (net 21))
 (segment (start 102.38 78.709275) (end 102.38 80.01) (width 0.25) (layer F.Cu) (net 21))
 (segment (start 102.38 77.47) (end 102.38 78.709275) (width 0.25) (layer F.Cu) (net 21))
 (segment (start 108.005 71.075) (end 108.005 76.125) (width 0.25) (layer F.Cu) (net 1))
 (segment (start 108.005 69.925) (end 108.005 71.075) (width 0.25) (layer F.Cu) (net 1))
 (segment (start 108.805 69.925) (end 108.005 69.925) (width 0.25) (layer F.Cu) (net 1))
 (segment (start 119.61499 75.47501) (end 119.61499 71.35499) (width 0.25) (layer F.Cu) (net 1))
 (segment (start 117.62 77.47) (end 119.61499 75.47501) (width 0.25) (layer F.Cu) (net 1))
 (segment (start 119.410001 71.150001) (end 119.61499 71.35499) (width 0.25) (layer F.Cu) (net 1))
 (segment (start 110.030001 71.150001) (end 119.410001 71.150001) (width 0.25) (layer F.Cu) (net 1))
 (segment (start 108.805 69.925) (end 110.030001 71.150001) (width 0.25) (layer F.Cu) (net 1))
 (segment (start 114.3 74.93) (end 117.62 74.93) (width 0.25) (layer F.Cu) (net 2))
 (segment (start 111.705 76.125) (end 111.705 75.775) (width 0.25) (layer F.Cu) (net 2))
 (segment (start 113.105 76.125) (end 114.3 74.93) (width 0.25) (layer F.Cu) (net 2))
 (segment (start 111.705 76.125) (end 113.105 76.125) (width 0.25) (layer F.Cu) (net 2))
 (segment (start 108.7375 80.01) (end 108.585 80.1625) (width 0.25) (layer F.Cu) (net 2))
 (segment (start 111.125 80.01) (end 108.7375 80.01) (width 0.25) (layer F.Cu) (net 2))
 (segment (start 108.01 80.1625) (end 107.315 79.4675) (width 0.25) (layer F.Cu) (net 2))
 (segment (start 108.585 80.1625) (end 108.01 80.1625) (width 0.25) (layer F.Cu) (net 2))
 (segment (start 107.315 79.4675) (end 107.315 78.105) (width 0.25) (layer F.Cu) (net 2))
 (segment (start 107.315 78.105) (end 107.95 77.47) (width 0.25) (layer F.Cu) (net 2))
 (segment (start 110.905 76.125) (end 111.705 76.125) (width 0.25) (layer F.Cu) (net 2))
 (segment (start 109.56 77.47) (end 110.905 76.125) (width 0.25) (layer F.Cu) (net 2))
 (segment (start 107.95 77.47) (end 109.56 77.47) (width 0.25) (layer F.Cu) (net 2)))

